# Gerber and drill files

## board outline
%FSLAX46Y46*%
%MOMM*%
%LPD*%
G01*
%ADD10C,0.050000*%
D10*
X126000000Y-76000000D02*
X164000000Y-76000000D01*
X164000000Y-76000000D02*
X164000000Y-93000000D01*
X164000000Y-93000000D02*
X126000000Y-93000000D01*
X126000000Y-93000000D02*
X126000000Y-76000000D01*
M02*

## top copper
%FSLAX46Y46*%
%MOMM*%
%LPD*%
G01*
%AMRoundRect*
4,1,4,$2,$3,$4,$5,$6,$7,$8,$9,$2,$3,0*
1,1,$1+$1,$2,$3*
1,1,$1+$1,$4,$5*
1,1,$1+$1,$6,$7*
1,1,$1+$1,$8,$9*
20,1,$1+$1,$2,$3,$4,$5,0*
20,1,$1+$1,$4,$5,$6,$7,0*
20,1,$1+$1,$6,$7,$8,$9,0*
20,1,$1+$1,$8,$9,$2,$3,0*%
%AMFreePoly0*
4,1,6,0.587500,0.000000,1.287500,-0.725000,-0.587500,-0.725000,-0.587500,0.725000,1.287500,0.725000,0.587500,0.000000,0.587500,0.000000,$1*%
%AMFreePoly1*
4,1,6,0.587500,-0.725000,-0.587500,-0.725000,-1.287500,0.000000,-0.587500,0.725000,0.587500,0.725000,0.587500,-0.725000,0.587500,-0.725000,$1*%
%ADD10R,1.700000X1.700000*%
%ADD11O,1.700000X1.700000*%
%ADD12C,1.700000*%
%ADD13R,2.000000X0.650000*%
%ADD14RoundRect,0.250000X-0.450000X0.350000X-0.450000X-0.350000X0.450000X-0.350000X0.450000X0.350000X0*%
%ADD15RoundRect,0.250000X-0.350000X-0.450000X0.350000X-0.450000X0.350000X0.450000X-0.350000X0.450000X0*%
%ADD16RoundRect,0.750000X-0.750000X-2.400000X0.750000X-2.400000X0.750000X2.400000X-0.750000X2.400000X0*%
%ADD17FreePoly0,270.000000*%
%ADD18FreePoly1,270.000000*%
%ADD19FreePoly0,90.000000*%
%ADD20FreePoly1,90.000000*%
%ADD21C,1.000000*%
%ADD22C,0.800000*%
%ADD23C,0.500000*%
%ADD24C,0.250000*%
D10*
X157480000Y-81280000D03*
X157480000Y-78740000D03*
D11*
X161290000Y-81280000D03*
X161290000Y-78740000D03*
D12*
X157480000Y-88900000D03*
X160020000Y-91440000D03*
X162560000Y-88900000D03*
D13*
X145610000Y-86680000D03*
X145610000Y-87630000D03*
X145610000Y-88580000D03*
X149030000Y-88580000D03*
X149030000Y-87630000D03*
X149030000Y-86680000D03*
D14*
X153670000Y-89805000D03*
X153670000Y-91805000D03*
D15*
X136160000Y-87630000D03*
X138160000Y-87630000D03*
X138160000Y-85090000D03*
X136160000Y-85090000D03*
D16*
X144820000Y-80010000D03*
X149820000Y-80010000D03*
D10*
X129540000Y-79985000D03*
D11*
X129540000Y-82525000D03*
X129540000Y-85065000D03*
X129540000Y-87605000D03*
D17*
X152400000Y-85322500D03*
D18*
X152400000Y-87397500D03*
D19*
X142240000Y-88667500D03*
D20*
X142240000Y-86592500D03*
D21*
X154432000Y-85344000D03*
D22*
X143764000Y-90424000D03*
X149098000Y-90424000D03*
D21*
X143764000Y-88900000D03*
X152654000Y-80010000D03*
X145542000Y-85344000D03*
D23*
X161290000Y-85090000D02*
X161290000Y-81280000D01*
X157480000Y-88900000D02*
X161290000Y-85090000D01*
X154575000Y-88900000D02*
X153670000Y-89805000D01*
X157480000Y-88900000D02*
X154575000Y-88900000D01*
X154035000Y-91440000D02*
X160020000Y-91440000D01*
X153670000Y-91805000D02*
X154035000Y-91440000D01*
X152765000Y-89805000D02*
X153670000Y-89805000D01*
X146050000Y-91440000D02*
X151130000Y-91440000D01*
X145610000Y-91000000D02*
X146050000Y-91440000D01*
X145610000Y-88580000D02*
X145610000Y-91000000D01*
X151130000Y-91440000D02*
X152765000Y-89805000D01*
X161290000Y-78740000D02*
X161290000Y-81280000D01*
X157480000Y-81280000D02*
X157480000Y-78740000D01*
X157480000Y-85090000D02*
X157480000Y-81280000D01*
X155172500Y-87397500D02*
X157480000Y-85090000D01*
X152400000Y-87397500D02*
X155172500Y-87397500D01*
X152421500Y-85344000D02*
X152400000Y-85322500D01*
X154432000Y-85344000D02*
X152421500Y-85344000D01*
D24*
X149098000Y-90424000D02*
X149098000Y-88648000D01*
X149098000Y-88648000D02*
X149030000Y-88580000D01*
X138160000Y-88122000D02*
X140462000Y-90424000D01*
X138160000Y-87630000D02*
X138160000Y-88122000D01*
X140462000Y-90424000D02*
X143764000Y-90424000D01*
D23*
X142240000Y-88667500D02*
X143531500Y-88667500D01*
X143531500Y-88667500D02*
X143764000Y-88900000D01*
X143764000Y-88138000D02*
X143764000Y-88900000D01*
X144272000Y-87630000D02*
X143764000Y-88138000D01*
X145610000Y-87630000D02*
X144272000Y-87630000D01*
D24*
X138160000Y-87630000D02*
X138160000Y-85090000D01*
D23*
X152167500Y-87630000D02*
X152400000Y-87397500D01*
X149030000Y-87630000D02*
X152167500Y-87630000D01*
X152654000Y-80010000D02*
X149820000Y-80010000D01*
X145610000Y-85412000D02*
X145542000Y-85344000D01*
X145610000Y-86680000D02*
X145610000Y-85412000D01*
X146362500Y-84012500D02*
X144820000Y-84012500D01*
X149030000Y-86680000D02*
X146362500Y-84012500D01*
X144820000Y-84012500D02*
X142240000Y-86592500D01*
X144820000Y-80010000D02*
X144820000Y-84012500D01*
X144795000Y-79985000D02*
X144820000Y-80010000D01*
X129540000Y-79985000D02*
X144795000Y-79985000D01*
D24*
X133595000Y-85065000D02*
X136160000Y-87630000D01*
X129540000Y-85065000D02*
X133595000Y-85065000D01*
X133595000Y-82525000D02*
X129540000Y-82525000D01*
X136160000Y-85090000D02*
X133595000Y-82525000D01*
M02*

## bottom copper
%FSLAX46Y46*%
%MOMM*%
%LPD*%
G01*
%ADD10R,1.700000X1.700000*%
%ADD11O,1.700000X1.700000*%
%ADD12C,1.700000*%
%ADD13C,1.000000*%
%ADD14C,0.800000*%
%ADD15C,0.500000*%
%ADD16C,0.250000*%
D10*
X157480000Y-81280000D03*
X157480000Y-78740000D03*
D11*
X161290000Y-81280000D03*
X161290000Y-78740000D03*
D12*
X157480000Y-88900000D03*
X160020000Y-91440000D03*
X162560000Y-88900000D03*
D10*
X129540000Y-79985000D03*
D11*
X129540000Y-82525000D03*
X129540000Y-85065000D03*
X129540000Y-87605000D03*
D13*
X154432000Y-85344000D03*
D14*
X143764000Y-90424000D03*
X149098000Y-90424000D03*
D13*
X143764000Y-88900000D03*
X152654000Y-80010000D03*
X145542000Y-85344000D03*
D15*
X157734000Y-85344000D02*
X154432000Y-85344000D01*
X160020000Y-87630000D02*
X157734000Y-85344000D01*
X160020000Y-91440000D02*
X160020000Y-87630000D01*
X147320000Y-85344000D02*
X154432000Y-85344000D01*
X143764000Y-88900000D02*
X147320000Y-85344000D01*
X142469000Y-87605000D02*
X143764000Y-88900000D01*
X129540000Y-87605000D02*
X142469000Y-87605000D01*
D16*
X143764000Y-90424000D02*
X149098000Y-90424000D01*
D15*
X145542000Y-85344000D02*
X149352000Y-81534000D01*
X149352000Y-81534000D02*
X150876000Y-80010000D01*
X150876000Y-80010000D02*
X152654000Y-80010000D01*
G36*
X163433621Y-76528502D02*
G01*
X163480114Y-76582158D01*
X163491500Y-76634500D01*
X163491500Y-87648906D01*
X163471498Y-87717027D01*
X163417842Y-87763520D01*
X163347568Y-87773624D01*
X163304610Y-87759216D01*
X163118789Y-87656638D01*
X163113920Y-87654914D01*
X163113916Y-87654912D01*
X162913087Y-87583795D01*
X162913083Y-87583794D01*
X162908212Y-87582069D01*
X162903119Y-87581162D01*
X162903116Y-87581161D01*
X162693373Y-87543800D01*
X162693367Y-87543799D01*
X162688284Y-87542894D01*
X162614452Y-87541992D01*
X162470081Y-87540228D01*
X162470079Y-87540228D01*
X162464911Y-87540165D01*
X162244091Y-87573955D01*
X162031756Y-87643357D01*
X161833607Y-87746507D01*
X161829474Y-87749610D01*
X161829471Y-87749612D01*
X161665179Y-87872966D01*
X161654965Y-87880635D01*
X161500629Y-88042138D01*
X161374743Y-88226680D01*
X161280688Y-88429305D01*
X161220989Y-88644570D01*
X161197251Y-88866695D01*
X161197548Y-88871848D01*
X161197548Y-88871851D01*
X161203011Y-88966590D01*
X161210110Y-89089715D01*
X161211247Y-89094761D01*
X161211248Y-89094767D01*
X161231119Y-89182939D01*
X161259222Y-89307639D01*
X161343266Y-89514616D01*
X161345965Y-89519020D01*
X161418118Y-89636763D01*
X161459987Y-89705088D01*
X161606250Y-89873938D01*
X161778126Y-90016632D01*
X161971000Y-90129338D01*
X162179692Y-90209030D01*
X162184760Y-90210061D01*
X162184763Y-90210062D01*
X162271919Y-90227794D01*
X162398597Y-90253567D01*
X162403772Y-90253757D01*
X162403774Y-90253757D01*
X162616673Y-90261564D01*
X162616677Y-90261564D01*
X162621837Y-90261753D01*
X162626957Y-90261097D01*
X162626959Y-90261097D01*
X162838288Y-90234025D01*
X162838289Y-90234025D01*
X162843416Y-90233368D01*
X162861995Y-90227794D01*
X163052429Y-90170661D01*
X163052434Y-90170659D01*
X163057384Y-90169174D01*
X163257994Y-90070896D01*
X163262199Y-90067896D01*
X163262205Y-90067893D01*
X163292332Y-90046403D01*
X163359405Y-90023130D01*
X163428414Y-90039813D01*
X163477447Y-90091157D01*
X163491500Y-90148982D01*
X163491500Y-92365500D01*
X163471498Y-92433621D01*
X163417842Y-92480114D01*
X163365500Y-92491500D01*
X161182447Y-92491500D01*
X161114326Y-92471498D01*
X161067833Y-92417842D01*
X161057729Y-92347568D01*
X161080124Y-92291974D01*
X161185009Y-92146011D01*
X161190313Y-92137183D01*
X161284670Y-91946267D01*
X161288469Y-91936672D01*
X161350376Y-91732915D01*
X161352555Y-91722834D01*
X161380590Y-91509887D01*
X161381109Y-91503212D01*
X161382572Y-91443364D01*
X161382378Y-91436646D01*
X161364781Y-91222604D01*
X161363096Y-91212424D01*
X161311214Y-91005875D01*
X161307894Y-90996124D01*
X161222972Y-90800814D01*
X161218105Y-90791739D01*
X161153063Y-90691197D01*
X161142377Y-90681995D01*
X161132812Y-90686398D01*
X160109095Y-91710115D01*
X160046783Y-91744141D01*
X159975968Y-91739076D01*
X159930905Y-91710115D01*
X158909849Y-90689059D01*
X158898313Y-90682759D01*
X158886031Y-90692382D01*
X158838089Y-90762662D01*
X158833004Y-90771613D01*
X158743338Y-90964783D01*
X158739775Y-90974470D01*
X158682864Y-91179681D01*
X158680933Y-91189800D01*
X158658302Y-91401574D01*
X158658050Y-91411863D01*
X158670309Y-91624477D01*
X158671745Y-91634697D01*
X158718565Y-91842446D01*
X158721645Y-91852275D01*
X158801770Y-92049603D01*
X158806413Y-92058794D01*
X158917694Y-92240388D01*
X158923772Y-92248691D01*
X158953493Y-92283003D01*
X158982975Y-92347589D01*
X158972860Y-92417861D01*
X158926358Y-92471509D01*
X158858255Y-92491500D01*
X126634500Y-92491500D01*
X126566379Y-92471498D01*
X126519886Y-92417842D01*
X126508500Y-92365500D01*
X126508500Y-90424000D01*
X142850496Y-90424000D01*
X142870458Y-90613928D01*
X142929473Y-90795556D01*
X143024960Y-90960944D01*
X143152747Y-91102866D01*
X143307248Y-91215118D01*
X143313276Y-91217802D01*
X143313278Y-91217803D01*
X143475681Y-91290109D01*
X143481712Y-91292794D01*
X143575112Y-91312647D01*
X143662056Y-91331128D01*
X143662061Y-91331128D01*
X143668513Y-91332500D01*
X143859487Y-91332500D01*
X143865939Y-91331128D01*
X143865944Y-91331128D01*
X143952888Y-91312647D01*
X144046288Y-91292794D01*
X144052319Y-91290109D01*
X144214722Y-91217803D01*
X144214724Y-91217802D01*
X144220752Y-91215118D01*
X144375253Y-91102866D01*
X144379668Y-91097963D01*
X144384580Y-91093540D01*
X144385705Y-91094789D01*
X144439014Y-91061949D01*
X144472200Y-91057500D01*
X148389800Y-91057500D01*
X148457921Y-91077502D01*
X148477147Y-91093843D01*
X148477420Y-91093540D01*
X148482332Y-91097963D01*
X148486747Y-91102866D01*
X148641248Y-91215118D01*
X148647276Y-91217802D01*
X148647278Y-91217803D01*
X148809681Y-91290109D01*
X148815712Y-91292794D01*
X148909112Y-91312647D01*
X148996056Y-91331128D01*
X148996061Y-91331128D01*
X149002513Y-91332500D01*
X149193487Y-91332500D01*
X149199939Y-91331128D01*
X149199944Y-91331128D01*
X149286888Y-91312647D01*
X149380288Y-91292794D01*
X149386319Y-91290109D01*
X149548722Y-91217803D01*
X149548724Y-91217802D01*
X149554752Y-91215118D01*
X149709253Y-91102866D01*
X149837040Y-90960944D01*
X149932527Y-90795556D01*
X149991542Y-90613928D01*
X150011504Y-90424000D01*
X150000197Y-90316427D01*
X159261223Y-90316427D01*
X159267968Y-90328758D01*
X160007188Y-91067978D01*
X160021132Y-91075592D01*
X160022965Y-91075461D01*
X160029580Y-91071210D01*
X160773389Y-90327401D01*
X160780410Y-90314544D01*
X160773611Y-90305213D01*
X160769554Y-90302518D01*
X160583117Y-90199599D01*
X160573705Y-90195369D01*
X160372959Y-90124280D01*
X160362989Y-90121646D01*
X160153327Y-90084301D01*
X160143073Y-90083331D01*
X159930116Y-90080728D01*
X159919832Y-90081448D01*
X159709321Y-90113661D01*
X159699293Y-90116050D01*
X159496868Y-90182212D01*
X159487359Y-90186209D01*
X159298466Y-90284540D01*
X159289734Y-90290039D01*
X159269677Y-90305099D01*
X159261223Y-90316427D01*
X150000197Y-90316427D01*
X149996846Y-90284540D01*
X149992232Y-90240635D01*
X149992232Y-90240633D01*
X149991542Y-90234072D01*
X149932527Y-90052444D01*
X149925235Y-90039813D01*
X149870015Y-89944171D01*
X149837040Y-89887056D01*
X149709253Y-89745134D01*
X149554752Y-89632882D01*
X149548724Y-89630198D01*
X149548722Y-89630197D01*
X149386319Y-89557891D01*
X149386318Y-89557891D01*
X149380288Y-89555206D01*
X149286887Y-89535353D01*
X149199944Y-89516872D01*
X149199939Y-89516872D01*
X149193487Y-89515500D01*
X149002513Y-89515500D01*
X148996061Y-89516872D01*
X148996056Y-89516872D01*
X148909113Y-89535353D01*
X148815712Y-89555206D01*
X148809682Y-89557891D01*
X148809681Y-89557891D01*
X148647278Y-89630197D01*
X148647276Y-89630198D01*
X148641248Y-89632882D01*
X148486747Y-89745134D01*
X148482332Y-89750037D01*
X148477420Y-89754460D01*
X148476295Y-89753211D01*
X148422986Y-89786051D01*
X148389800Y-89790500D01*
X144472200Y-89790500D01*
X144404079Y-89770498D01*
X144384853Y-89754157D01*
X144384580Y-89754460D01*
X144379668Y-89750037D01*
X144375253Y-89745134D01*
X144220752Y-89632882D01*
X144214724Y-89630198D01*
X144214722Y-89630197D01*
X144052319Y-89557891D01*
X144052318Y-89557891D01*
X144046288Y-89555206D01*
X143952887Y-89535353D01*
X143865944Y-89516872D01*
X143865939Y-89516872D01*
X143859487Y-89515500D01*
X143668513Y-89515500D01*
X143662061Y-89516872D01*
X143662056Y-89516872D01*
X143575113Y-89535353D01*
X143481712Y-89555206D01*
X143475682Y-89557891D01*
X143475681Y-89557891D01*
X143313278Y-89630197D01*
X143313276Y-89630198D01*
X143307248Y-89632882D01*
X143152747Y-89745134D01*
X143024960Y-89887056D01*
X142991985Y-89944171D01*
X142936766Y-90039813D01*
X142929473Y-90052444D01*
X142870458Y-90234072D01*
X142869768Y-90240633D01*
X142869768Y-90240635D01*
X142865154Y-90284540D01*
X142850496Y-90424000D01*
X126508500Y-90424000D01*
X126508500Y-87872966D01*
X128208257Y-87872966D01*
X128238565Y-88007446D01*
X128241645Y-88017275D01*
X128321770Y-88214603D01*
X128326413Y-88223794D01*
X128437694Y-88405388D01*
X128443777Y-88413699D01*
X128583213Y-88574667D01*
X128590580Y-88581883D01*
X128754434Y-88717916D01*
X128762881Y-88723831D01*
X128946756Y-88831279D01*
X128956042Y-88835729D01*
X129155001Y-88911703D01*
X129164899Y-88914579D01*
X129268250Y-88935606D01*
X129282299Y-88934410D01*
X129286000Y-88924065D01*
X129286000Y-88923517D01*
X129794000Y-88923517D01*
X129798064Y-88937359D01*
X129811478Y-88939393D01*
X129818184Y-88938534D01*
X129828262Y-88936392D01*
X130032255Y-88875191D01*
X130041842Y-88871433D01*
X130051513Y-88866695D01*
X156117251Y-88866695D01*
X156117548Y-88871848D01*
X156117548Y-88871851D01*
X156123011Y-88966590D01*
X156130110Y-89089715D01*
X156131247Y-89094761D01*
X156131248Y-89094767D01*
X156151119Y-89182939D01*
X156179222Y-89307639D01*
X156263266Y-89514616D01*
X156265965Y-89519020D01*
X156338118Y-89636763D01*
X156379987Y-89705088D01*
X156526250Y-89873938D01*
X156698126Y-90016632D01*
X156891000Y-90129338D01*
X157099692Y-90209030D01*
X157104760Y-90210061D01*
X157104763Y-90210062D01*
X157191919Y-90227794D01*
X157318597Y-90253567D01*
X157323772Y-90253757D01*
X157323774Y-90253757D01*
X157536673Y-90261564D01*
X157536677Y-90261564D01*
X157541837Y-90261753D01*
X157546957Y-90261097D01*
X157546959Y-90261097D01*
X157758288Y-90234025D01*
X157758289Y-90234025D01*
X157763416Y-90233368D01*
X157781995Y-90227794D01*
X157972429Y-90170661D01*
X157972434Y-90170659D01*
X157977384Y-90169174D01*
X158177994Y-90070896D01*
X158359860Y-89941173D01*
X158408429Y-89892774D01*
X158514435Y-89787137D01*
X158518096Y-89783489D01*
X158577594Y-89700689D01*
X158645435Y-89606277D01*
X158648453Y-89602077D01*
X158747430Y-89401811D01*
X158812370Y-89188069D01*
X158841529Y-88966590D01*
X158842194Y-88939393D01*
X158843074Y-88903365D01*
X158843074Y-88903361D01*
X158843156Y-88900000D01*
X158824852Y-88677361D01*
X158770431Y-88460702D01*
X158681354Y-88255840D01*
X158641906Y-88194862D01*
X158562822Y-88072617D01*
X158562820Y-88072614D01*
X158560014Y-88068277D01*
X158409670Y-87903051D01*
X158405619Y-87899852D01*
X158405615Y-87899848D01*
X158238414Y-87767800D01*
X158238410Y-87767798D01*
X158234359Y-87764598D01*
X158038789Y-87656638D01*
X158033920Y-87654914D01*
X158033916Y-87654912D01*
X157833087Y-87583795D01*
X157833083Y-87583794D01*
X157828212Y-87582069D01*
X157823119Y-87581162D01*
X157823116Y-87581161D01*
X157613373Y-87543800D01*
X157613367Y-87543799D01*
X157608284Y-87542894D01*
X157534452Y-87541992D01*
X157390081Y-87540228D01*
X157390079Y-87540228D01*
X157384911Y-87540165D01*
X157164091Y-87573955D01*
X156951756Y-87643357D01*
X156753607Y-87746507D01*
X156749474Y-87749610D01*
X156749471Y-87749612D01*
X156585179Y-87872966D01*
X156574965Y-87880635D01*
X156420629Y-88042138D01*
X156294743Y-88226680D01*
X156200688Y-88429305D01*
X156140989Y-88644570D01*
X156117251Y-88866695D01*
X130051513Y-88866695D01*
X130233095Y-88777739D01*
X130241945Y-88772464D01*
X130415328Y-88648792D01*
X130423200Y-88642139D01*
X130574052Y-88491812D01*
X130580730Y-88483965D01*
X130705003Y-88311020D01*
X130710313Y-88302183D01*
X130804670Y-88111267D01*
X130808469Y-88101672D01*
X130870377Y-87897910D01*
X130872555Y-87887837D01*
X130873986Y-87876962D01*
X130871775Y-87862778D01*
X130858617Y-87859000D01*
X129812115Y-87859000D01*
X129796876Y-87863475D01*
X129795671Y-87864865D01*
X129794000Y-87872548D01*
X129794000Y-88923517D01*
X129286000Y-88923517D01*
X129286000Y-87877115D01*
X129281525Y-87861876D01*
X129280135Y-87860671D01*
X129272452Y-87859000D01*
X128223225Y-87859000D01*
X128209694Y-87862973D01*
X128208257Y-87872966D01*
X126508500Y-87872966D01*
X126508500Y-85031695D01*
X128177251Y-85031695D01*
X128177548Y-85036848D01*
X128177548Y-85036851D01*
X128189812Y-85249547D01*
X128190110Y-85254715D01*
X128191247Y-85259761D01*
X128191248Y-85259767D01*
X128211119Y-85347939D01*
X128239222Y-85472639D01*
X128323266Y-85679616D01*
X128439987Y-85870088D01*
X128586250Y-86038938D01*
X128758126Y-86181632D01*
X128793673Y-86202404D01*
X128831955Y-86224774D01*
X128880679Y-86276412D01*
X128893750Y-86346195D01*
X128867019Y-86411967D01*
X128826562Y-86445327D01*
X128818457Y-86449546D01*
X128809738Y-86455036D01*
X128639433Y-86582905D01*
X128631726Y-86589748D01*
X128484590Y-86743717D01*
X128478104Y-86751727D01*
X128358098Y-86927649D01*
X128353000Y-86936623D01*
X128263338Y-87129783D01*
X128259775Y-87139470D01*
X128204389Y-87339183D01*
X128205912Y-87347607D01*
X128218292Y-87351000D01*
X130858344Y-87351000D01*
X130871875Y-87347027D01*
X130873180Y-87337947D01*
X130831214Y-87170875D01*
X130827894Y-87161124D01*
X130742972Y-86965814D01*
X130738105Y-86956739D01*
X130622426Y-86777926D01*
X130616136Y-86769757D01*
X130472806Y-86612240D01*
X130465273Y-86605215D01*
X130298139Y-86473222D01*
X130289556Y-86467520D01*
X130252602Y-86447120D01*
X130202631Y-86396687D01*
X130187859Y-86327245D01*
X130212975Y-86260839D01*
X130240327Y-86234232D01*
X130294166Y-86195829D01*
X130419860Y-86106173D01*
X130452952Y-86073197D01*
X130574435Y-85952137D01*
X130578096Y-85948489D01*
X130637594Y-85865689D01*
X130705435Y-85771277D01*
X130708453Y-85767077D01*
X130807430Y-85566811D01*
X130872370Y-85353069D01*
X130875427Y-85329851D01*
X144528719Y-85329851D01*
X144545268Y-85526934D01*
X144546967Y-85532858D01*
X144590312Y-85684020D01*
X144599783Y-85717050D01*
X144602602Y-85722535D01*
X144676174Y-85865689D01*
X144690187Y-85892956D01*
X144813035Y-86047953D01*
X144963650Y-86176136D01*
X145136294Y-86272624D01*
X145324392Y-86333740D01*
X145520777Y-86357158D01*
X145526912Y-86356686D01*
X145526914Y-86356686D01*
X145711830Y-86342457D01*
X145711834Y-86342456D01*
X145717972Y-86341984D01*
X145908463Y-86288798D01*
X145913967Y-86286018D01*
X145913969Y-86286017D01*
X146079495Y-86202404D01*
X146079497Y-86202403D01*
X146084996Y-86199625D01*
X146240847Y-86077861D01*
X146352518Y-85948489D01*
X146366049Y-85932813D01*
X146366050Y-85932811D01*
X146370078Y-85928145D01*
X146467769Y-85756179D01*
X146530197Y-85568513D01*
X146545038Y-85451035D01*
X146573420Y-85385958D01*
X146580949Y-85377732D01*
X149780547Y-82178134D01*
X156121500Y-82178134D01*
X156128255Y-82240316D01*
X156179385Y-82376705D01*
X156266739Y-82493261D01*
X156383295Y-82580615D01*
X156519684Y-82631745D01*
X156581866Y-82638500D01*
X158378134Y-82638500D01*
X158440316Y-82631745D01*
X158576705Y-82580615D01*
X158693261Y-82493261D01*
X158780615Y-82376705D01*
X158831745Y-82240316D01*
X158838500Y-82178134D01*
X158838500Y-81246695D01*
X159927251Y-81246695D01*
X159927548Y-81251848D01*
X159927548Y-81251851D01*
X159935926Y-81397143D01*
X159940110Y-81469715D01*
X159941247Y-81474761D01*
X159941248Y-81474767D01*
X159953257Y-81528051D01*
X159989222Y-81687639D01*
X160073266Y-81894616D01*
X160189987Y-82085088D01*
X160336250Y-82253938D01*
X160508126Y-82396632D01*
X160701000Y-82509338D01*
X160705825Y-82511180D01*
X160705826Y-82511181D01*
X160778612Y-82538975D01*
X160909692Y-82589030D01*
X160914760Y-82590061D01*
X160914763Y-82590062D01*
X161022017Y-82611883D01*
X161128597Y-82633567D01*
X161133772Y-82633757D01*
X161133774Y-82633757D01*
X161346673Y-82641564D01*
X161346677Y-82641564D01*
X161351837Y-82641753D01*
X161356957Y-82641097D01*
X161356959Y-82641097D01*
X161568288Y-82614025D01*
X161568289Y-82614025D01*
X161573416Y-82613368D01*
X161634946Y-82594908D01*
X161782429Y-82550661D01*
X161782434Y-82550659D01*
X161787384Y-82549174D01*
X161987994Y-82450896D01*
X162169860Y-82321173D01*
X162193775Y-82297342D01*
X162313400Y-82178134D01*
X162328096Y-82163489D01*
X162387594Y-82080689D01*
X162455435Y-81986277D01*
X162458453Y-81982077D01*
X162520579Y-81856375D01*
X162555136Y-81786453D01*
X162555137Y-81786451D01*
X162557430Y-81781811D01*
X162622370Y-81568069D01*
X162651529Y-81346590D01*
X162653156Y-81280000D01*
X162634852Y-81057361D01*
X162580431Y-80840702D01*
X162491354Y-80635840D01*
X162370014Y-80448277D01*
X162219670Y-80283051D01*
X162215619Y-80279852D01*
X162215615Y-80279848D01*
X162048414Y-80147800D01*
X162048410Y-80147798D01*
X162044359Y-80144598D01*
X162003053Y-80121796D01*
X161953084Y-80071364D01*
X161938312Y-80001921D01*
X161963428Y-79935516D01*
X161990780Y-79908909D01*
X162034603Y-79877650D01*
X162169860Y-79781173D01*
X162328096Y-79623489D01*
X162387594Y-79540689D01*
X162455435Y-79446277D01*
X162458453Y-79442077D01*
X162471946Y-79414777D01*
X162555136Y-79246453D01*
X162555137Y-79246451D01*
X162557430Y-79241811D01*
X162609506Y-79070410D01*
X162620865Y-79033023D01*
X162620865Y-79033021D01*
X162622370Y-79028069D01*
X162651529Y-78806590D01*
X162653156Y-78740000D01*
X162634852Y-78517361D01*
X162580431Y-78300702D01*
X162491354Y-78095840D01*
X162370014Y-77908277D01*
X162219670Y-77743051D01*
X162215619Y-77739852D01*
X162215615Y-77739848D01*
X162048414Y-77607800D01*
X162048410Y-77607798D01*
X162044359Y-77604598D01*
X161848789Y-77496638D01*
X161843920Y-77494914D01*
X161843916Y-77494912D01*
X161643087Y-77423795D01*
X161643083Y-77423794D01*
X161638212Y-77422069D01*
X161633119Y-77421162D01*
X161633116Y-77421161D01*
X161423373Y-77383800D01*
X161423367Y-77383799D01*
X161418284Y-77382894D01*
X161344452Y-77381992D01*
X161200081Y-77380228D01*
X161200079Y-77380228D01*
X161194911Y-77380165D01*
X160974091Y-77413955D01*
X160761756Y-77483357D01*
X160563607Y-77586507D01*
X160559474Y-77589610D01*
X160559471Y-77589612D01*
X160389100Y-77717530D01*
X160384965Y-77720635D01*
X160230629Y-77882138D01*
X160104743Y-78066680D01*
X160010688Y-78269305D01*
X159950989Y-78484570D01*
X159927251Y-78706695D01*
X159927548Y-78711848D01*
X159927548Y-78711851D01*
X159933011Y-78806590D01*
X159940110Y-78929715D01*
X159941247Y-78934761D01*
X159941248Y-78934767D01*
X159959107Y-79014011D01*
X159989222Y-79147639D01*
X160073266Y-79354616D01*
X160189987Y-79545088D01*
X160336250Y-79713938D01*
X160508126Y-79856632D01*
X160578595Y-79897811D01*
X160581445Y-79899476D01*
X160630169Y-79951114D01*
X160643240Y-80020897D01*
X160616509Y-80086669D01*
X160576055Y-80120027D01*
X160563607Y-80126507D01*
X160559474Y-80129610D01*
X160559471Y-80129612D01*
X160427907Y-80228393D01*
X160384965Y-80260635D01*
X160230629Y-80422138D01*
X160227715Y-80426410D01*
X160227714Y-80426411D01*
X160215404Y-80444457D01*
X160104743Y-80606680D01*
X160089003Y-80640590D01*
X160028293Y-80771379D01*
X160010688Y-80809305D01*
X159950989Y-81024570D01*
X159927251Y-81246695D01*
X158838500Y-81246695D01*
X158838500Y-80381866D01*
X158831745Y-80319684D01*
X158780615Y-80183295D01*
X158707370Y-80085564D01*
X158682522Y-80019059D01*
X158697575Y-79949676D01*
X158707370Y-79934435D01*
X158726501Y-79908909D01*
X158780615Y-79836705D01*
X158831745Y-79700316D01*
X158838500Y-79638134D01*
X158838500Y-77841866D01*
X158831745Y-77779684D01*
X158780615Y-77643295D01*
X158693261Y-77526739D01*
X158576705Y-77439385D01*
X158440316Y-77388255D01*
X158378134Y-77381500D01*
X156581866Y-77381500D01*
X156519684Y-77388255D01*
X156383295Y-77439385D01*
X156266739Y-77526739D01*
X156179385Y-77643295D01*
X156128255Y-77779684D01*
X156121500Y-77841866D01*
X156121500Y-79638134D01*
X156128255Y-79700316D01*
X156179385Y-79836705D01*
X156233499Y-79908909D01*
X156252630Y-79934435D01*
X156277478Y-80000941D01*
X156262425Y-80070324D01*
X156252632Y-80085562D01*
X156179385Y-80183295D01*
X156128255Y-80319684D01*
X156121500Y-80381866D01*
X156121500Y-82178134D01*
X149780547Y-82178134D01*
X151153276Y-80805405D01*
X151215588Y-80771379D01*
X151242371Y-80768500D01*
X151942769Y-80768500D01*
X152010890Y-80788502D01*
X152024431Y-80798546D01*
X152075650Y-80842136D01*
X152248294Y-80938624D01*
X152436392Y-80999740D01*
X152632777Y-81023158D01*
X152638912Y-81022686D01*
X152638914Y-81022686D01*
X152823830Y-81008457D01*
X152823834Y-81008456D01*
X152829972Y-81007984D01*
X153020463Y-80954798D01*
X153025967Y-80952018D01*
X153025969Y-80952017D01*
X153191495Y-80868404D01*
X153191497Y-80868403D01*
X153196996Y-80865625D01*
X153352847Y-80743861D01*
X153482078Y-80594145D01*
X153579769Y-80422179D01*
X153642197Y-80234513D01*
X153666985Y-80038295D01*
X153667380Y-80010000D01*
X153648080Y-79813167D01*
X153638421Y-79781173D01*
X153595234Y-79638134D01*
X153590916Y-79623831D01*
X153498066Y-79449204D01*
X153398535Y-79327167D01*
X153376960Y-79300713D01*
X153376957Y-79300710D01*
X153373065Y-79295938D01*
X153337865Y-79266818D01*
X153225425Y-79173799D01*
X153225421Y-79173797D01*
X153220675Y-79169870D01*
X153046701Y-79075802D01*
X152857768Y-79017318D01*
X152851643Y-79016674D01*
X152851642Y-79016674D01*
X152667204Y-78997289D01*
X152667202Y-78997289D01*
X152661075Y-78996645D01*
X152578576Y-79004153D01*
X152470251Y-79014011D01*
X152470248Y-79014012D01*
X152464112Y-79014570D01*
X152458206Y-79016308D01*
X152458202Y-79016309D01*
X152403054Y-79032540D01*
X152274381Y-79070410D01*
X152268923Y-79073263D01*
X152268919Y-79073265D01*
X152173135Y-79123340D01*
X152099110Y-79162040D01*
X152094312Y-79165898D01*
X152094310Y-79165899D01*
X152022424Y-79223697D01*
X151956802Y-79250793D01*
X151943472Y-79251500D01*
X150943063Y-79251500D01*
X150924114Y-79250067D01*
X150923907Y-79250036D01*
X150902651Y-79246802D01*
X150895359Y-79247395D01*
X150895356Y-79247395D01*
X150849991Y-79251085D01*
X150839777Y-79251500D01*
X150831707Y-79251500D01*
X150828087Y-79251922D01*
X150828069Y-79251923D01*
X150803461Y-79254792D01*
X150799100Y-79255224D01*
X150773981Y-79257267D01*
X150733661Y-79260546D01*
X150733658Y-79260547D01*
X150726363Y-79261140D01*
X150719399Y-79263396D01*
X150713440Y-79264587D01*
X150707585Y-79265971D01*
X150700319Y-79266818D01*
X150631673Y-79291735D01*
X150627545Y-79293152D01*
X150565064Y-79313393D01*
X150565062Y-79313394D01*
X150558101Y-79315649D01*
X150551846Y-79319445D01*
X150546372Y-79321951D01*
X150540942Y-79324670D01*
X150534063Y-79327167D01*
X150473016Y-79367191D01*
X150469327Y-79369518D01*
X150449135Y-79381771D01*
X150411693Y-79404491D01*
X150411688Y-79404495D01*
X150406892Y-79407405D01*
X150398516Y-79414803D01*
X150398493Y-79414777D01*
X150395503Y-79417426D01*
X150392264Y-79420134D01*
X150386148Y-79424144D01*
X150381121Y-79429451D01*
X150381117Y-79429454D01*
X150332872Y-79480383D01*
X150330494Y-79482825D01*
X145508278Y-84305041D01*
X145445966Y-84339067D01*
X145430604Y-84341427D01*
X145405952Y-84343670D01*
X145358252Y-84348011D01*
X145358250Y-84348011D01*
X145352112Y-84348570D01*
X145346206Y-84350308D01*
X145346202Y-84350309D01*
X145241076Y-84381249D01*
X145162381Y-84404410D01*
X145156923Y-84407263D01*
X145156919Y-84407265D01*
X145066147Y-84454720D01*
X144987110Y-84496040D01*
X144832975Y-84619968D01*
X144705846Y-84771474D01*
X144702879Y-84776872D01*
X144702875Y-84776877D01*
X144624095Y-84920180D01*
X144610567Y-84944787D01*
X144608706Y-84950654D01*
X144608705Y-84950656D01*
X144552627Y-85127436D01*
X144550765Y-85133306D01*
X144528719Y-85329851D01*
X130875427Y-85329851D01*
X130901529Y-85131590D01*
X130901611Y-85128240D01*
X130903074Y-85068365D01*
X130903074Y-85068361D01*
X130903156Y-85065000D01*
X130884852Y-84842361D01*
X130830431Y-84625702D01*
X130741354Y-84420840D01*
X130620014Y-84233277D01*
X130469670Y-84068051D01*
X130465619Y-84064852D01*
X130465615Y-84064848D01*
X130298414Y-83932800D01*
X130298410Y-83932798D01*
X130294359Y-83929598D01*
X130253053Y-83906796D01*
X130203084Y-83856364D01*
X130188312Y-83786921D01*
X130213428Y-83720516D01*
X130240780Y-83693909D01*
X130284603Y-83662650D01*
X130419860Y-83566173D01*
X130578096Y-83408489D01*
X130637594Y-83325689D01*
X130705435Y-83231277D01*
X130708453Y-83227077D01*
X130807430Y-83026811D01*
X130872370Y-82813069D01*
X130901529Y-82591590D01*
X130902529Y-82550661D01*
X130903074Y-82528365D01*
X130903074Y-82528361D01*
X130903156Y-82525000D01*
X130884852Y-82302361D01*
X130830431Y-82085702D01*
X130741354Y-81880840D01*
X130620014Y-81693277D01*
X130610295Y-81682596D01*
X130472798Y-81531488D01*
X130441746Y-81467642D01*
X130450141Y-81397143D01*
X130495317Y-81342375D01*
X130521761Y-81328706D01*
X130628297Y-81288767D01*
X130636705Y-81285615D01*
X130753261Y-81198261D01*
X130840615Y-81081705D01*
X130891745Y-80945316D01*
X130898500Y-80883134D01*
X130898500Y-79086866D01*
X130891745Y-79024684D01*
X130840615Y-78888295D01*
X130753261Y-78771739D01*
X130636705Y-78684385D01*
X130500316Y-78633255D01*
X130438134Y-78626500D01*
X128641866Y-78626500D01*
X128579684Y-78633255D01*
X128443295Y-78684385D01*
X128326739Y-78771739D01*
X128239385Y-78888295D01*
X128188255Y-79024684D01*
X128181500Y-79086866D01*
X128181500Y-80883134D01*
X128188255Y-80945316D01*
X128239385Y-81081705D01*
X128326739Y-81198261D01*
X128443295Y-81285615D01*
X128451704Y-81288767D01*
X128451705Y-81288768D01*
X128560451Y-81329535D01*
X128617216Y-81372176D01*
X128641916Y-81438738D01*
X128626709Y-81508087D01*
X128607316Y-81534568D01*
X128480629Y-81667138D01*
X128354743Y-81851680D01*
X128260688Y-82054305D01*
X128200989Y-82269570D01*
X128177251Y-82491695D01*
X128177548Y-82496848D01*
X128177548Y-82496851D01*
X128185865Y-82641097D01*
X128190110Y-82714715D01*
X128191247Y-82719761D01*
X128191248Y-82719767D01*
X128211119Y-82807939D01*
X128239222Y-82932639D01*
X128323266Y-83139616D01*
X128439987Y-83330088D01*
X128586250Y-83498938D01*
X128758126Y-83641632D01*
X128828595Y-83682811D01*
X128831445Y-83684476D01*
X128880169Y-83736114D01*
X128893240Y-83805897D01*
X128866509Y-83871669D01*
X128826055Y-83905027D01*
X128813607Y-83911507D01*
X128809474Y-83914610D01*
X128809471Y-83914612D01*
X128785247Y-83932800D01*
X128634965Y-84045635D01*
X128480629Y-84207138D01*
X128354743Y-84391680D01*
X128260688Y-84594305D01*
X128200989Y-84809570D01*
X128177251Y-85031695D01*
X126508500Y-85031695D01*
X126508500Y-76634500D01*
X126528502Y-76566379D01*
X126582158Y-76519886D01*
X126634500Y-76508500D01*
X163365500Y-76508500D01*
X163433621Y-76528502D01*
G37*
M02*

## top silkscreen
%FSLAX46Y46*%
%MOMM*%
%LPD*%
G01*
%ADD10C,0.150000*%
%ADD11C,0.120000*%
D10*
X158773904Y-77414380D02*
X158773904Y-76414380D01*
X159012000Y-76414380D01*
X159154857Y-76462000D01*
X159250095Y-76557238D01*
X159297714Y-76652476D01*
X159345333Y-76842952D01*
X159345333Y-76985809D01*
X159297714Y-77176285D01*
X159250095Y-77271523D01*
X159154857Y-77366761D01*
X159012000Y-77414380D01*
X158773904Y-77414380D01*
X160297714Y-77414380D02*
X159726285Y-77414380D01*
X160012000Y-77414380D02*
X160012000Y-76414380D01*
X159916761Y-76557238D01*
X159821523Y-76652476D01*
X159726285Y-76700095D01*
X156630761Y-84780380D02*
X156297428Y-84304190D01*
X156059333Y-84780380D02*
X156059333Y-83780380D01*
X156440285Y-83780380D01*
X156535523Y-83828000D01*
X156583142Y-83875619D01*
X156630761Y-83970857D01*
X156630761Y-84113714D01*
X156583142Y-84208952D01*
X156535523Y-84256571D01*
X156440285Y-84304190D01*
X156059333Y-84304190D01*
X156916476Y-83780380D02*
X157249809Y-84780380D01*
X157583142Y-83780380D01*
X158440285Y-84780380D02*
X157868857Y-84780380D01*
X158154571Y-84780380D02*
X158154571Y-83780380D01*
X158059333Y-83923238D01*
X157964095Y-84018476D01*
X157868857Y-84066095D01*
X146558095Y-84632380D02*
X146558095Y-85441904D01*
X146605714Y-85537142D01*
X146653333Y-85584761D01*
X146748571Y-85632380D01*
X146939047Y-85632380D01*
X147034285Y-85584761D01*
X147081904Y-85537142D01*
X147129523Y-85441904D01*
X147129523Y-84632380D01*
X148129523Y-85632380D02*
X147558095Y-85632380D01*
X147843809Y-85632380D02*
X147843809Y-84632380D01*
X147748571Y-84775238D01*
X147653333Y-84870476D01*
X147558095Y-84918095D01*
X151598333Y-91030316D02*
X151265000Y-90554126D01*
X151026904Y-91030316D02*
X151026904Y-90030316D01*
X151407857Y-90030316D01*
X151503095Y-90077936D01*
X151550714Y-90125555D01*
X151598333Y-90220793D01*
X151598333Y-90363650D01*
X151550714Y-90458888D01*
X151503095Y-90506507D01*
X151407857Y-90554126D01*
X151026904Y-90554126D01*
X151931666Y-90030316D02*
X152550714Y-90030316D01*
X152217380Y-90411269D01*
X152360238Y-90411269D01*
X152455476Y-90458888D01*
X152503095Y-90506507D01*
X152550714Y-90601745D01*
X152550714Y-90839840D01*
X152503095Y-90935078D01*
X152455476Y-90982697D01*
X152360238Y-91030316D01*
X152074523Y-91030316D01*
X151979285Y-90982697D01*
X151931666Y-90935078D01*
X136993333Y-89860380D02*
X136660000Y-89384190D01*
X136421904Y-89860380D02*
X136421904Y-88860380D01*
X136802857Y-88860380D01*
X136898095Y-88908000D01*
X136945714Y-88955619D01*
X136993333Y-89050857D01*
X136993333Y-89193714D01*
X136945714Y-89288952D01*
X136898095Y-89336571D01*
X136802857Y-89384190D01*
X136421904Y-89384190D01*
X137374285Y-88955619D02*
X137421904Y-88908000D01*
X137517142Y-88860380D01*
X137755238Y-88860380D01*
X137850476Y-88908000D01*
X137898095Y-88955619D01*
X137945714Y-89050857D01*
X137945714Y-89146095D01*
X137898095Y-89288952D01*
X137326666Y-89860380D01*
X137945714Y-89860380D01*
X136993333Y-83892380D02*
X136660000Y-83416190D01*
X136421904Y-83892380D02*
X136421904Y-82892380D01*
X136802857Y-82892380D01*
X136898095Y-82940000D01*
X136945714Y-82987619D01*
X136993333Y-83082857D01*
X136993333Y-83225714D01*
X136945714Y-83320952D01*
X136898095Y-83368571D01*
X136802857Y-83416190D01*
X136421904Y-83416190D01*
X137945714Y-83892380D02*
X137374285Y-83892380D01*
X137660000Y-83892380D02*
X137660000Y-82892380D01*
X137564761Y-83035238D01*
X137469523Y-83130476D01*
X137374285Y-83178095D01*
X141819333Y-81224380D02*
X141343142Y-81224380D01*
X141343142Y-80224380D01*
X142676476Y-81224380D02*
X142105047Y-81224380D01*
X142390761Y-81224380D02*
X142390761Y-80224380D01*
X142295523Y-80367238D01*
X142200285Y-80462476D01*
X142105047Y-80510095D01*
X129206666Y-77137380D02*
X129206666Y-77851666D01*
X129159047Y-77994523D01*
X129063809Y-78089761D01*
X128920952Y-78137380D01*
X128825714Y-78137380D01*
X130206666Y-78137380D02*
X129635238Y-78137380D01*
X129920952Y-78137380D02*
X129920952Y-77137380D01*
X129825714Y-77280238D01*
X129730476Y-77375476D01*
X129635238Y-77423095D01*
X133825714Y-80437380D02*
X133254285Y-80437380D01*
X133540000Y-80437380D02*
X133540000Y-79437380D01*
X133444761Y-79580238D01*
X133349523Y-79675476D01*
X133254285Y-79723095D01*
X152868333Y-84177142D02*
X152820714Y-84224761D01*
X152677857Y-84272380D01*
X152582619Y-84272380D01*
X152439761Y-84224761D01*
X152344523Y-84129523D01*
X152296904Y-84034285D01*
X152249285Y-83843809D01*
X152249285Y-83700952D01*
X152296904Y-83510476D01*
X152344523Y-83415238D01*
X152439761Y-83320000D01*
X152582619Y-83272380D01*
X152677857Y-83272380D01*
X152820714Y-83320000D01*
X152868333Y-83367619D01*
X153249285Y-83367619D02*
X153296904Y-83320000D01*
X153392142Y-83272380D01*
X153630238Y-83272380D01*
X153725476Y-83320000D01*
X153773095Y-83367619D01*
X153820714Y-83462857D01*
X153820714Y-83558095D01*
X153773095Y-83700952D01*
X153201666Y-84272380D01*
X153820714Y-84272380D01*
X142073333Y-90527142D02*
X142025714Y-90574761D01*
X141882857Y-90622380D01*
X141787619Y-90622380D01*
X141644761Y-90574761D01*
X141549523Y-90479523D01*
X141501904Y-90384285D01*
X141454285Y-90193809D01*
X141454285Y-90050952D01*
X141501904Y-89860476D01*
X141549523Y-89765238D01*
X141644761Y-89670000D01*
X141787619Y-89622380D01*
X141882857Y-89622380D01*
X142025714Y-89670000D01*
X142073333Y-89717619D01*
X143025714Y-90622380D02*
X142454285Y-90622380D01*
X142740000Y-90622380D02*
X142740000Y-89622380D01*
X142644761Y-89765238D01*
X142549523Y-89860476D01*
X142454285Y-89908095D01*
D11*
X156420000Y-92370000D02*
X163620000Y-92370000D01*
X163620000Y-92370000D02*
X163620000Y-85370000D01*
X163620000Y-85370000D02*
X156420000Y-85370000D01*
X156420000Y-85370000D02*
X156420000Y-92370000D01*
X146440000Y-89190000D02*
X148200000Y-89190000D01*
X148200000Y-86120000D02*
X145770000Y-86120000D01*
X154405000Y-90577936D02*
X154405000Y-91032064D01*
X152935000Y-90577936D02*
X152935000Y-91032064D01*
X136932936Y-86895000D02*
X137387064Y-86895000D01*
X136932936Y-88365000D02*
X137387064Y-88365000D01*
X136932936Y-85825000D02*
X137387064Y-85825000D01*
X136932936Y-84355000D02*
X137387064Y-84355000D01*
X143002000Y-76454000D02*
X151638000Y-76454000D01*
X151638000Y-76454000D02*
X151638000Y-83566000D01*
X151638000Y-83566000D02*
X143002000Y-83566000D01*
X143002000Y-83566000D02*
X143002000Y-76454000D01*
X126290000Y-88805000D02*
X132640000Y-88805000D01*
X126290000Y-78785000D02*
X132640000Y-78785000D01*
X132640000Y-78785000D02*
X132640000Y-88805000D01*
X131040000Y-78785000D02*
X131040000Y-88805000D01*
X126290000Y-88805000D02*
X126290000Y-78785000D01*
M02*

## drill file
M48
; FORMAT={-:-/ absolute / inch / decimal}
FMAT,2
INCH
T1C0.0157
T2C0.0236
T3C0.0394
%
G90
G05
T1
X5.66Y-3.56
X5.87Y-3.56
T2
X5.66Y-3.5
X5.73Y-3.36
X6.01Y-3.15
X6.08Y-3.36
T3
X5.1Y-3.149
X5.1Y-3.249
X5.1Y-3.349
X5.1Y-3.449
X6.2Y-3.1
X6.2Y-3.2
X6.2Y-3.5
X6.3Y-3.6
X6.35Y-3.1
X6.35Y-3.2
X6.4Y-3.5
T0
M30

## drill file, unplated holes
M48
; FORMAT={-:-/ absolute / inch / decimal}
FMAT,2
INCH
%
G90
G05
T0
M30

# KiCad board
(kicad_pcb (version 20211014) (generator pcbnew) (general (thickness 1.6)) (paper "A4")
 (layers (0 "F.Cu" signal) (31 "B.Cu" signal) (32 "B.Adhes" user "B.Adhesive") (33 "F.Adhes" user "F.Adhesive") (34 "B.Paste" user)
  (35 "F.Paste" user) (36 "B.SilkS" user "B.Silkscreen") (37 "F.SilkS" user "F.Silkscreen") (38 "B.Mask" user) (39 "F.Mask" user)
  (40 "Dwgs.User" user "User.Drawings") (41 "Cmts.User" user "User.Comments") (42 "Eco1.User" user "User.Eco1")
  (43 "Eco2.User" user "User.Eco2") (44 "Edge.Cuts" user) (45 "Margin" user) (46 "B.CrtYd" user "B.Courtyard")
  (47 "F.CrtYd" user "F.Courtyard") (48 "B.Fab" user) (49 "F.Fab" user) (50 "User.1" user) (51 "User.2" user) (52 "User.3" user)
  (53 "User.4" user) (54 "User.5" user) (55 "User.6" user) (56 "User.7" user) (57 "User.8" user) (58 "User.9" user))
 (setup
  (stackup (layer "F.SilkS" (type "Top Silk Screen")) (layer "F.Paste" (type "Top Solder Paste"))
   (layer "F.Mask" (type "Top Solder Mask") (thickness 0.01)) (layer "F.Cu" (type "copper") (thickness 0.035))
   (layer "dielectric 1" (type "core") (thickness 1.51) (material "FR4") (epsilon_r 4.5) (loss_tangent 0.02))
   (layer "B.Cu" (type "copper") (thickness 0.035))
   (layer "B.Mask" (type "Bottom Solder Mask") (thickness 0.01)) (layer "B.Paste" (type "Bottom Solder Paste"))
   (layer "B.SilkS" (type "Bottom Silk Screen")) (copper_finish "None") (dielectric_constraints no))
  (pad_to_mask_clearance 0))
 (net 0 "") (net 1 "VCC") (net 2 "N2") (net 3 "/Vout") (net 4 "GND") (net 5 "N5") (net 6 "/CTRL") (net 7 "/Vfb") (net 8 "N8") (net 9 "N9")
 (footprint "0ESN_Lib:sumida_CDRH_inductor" (layer "F.Cu") (at 147.32 80.01)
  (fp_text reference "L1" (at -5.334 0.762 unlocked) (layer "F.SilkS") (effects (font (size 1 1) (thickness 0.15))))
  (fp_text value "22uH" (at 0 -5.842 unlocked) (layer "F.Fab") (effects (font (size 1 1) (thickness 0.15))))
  (fp_rect (start -4.318 -3.556) (end 4.318 3.556) (layer "F.SilkS") (width 0.12) (fill none))
  (pad "1" smd roundrect (at -2.5 0) (size 3 6.3) (layers "F.Cu" "F.Paste" "F.Mask") (roundrect_rratio 0.25) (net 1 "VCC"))
  (pad "2" smd roundrect (at 2.5 0) (size 3 6.3) (layers "F.Cu" "F.Paste" "F.Mask") (roundrect_rratio 0.25) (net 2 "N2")))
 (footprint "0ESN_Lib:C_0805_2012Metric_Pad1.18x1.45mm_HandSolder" (layer "F.Cu") (at 152.4 86.36 90)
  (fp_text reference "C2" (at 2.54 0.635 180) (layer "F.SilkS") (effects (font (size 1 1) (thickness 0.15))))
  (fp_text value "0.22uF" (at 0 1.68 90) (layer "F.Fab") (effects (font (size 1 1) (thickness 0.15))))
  (pad "1" smd custom (at -1.0375 0 270) (size 1.175 1.45) (layers "F.Cu" "F.Paste" "F.Mask") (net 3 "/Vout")
   (options (clearance outline) (anchor rect)) (primitives))
  (pad "2" smd custom (at 1.0375 0 270) (size 1.175 1.45) (layers "F.Cu" "F.Paste" "F.Mask") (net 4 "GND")
   (options (clearance outline) (anchor rect)) (primitives)))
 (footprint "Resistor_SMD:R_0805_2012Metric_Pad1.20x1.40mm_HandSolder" (layer "F.Cu") (at 137.16 87.63)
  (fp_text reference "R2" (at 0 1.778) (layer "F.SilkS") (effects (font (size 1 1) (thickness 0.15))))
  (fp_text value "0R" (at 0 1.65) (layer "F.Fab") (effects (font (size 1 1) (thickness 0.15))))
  (fp_line (start -0.227064 0.735) (end 0.227064 0.735) (layer "F.SilkS") (width 0.12))
  (fp_line (start -0.227064 -0.735) (end 0.227064 -0.735) (layer "F.SilkS") (width 0.12))
  (pad "1" smd roundrect (at -1 0) (size 1.2 1.4) (layers "F.Cu" "F.Paste" "F.Mask") (roundrect_rratio 0.2083333333) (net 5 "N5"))
  (pad "2" smd roundrect (at 1 0) (size 1.2 1.4) (layers "F.Cu" "F.Paste" "F.Mask") (roundrect_rratio 0.2083333333) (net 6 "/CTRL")))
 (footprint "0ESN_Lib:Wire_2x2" (layer "F.Cu") (at 158.75 81.28 90)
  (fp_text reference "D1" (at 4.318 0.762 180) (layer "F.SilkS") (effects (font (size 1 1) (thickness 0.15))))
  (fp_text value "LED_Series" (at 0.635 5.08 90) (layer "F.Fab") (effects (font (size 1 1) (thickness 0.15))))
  (pad "1" thru_hole rect (at 0 -1.27 90) (size 1.7 1.7) (drill 1) (layers *.Cu *.Mask) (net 3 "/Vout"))
  (pad "1" thru_hole rect (at 2.54 -1.27 90) (size 1.7 1.7) (drill 1) (layers *.Cu *.Mask) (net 3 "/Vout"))
  (pad "2" thru_hole oval (at 2.54 2.54 90) (size 1.7 1.7) (drill 1) (layers *.Cu *.Mask) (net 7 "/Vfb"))
  (pad "2" thru_hole oval (at 0 2.54 90) (size 1.7 1.7) (drill 1) (layers *.Cu *.Mask) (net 7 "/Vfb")))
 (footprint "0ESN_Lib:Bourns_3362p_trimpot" (layer "F.Cu") (at 160.02 88.9)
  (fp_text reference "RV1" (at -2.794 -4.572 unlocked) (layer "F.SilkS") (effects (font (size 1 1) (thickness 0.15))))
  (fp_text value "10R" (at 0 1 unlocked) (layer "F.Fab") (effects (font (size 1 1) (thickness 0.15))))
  (fp_rect (start -3.6 3.47) (end 3.6 -3.53) (layer "F.SilkS") (width 0.12) (fill none))
  (pad "1" thru_hole circle (at -2.54 0) (size 1.7 1.7) (drill 1) (layers *.Cu *.Mask) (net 7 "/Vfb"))
  (pad "2" thru_hole circle (at 0 2.54) (size 1.7 1.7) (drill 1) (layers *.Cu *.Mask) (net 4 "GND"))
  (pad "3" thru_hole circle (at 2.54 0) (size 1.7 1.7) (drill 1) (layers *.Cu *.Mask) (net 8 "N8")))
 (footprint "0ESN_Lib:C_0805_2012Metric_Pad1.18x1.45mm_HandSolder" (layer "F.Cu") (at 142.24 87.63 -90)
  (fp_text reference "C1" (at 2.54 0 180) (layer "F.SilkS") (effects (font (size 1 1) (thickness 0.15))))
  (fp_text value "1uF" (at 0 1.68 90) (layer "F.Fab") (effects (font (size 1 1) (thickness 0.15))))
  (pad "1" smd custom (at -1.0375 0 90) (size 1.175 1.45) (layers "F.Cu" "F.Paste" "F.Mask") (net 1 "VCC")
   (options (clearance outline) (anchor rect)) (primitives))
  (pad "2" smd custom (at 1.0375 0 90) (size 1.175 1.45) (layers "F.Cu" "F.Paste" "F.Mask") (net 4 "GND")
   (options (clearance outline) (anchor rect)) (primitives)))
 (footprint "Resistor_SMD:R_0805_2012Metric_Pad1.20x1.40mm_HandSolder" (layer "F.Cu") (at 153.67 90.805 -90)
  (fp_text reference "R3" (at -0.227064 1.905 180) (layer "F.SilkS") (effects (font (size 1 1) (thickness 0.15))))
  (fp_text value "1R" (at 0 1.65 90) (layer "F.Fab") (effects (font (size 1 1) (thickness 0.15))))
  (fp_line (start -0.227064 -0.735) (end 0.227064 -0.735) (layer "F.SilkS") (width 0.12))
  (fp_line (start -0.227064 0.735) (end 0.227064 0.735) (layer "F.SilkS") (width 0.12))
  (pad "1" smd roundrect (at -1 0 270) (size 1.2 1.4) (layers "F.Cu" "F.Paste" "F.Mask") (roundrect_rratio 0.2083333333) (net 7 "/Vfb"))
  (pad "2" smd roundrect (at 1 0 270) (size 1.2 1.4) (layers "F.Cu" "F.Paste" "F.Mask") (roundrect_rratio 0.2083333333) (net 4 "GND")))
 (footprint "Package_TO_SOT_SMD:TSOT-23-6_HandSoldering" (layer "F.Cu") (at 147.32 87.63)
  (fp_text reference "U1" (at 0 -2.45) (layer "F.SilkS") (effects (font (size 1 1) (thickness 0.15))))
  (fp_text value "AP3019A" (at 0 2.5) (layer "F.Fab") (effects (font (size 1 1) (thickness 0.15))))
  (fp_line (start 0.88 -1.51) (end -1.55 -1.51) (layer "F.SilkS") (width 0.12))
  (fp_line (start -0.88 1.56) (end 0.88 1.56) (layer "F.SilkS") (width 0.12))
  (pad "1" smd rect (at -1.71 -0.95) (size 2 0.65) (layers "F.Cu" "F.Paste" "F.Mask") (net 2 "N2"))
  (pad "2" smd rect (at -1.71 0) (size 2 0.65) (layers "F.Cu" "F.Paste" "F.Mask") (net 4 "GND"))
  (pad "3" smd rect (at -1.71 0.95) (size 2 0.65) (layers "F.Cu" "F.Paste" "F.Mask") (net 7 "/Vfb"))
  (pad "4" smd rect (at 1.71 0.95) (size 2 0.65) (layers "F.Cu" "F.Paste" "F.Mask") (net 6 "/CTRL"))
  (pad "5" smd rect (at 1.71 0) (size 2 0.65) (layers "F.Cu" "F.Paste" "F.Mask") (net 3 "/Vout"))
  (pad "6" smd rect (at 1.71 -0.95) (size 2 0.65) (layers "F.Cu" "F.Paste" "F.Mask") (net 1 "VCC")))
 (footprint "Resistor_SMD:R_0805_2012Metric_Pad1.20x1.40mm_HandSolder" (layer "F.Cu") (at 137.16 85.09)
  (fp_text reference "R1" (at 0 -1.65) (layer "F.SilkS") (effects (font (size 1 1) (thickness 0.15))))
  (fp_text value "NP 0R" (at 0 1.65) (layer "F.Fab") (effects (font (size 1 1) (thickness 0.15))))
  (fp_line (start -0.227064 0.735) (end 0.227064 0.735) (layer "F.SilkS") (width 0.12))
  (fp_line (start -0.227064 -0.735) (end 0.227064 -0.735) (layer "F.SilkS") (width 0.12))
  (pad "1" smd roundrect (at -1 0) (size 1.2 1.4) (layers "F.Cu" "F.Paste" "F.Mask") (roundrect_rratio 0.2083333333) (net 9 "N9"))
  (pad "2" smd roundrect (at 1 0) (size 1.2 1.4) (layers "F.Cu" "F.Paste" "F.Mask") (roundrect_rratio 0.2083333333) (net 6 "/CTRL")))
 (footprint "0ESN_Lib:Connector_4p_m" (layer "F.Cu") (at 129.54 79.985)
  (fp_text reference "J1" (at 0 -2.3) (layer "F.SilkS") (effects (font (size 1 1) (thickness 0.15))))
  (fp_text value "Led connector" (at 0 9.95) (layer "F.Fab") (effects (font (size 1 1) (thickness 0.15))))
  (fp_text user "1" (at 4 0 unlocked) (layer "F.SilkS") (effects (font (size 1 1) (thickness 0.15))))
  (fp_line (start 1.5 -1.2) (end 1.5 8.82) (layer "F.SilkS") (width 0.12))
  (fp_line (start -3.25 8.82) (end -3.25 -1.2) (layer "F.SilkS") (width 0.12))
  (fp_line (start 3.1 -1.2) (end 3.1 8.82) (layer "F.SilkS") (width 0.12))
  (fp_line (start -3.25 -1.2) (end 3.1 -1.2) (layer "F.SilkS") (width 0.12))
  (fp_line (start -3.25 8.82) (end 3.1 8.82) (layer "F.SilkS") (width 0.12))
  (pad "1" thru_hole rect (at 0 0) (size 1.7 1.7) (drill 1) (layers *.Cu *.Mask) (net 1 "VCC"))
  (pad "2" thru_hole oval (at 0 2.54) (size 1.7 1.7) (drill 1) (layers *.Cu *.Mask) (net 9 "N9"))
  (pad "3" thru_hole oval (at 0 5.08) (size 1.7 1.7) (drill 1) (layers *.Cu *.Mask) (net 5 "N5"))
  (pad "4" thru_hole oval (at 0 7.62) (size 1.7 1.7) (drill 1) (layers *.Cu *.Mask) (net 4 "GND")))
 (gr_rect (start 126 76) (end 164 93) (layer "Edge.Cuts") (width 0.05) (fill none))
 (segment (start 129.54 79.985) (end 144.795 79.985) (width 0.5) (layer "F.Cu") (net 1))
 (segment (start 144.795 79.985) (end 144.82 80.01) (width 0.5) (layer "F.Cu") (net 1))
 (segment (start 149.03 86.68) (end 146.3625 84.0125) (width 0.5) (layer "F.Cu") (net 1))
 (segment (start 144.82 80.01) (end 144.82 84.0125) (width 0.5) (layer "F.Cu") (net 1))
 (segment (start 144.82 84.0125) (end 142.24 86.5925) (width 0.5) (layer "F.Cu") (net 1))
 (segment (start 146.3625 84.0125) (end 144.82 84.0125) (width 0.5) (layer "F.Cu") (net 1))
 (segment (start 154.035 91.44) (end 160.02 91.44) (width 0.5) (layer "F.Cu") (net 4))
 (segment (start 152.4215 85.344) (end 152.4 85.3225) (width 0.5) (layer "F.Cu") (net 4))
 (segment (start 145.61 87.63) (end 144.272 87.63) (width 0.5) (layer "F.Cu") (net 4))
 (segment (start 154.432 85.344) (end 152.4215 85.344) (width 0.5) (layer "F.Cu") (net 4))
 (segment (start 142.24 88.6675) (end 143.5315 88.6675) (width 0.5) (layer "F.Cu") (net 4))
 (segment (start 143.5315 88.6675) (end 143.764 88.9) (width 0.5) (layer "F.Cu") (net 4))
 (segment (start 153.67 91.805) (end 154.035 91.44) (width 0.5) (layer "F.Cu") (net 4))
 (segment (start 144.272 87.63) (end 143.764 88.138) (width 0.5) (layer "F.Cu") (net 4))
 (segment (start 143.764 88.138) (end 143.764 88.9) (width 0.5) (layer "F.Cu") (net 4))
 (via (at 143.764 88.9) (size 1) (drill 0.6) (layers "F.Cu" "B.Cu") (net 4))
 (via (at 154.432 85.344) (size 1) (drill 0.6) (layers "F.Cu" "B.Cu") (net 4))
 (segment (start 147.32 85.344) (end 154.432 85.344) (width 0.5) (layer "B.Cu") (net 4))
 (segment (start 157.734 85.344) (end 154.432 85.344) (width 0.5) (layer "B.Cu") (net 4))
 (segment (start 160.02 87.63) (end 157.734 85.344) (width 0.5) (layer "B.Cu") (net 4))
 (segment (start 142.469 87.605) (end 143.764 88.9) (width 0.5) (layer "B.Cu") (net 4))
 (segment (start 143.764 88.9) (end 147.32 85.344) (width 0.5) (layer "B.Cu") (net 4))
 (segment (start 129.54 87.605) (end 142.469 87.605) (width 0.5) (layer "B.Cu") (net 4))
 (segment (start 160.02 91.44) (end 160.02 87.63) (width 0.5) (layer "B.Cu") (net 4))
 (segment (start 152.4 87.3975) (end 155.1725 87.3975) (width 0.5) (layer "F.Cu") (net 3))
 (segment (start 157.48 81.28) (end 157.48 78.74) (width 0.5) (layer "F.Cu") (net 3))
 (segment (start 157.48 85.09) (end 157.48 81.28) (width 0.5) (layer "F.Cu") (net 3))
 (segment (start 155.1725 87.3975) (end 157.48 85.09) (width 0.5) (layer "F.Cu") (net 3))
 (segment (start 149.03 87.63) (end 152.1675 87.63) (width 0.5) (layer "F.Cu") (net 3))
 (segment (start 152.1675 87.63) (end 152.4 87.3975) (width 0.5) (layer "F.Cu") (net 3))
 (segment (start 157.48 88.9) (end 161.29 85.09) (width 0.5) (layer "F.Cu") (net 7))
 (segment (start 146.05 91.44) (end 151.13 91.44) (width 0.5) (layer "F.Cu") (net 7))
 (segment (start 145.61 91) (end 146.05 91.44) (width 0.5) (layer "F.Cu") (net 7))
 (segment (start 151.13 91.44) (end 152.765 89.805) (width 0.5) (layer "F.Cu") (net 7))
 (segment (start 154.575 88.9) (end 153.67 89.805) (width 0.5) (layer "F.Cu") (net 7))
 (segment (start 145.61 88.58) (end 145.61 91) (width 0.5) (layer "F.Cu") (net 7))
 (segment (start 152.765 89.805) (end 153.67 89.805) (width 0.5) (layer "F.Cu") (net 7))
 (segment (start 161.29 85.09) (end 161.29 81.28) (width 0.5) (layer "F.Cu") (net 7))
 (segment (start 161.29 78.74) (end 161.29 81.28) (width 0.5) (layer "F.Cu") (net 7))
 (segment (start 157.48 88.9) (end 154.575 88.9) (width 0.5) (layer "F.Cu") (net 7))
 (segment (start 136.16 85.09) (end 133.595 82.525) (width 0.25) (layer "F.Cu") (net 9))
 (segment (start 133.595 82.525) (end 129.54 82.525) (width 0.25) (layer "F.Cu") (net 9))
 (segment (start 133.595 85.065) (end 136.16 87.63) (width 0.25) (layer "F.Cu") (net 5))
 (segment (start 129.54 85.065) (end 133.595 85.065) (width 0.25) (layer "F.Cu") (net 5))
 (segment (start 145.61 86.68) (end 145.61 85.412) (width 0.5) (layer "F.Cu") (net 2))
 (segment (start 145.61 85.412) (end 145.542 85.344) (width 0.5) (layer "F.Cu") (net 2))
 (segment (start 152.654 80.01) (end 149.82 80.01) (width 0.5) (layer "F.Cu") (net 2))
 (via (at 145.542 85.344) (size 1) (drill 0.6) (layers "F.Cu" "B.Cu") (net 2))
 (via (at 152.654 80.01) (size 1) (drill 0.6) (layers "F.Cu" "B.Cu") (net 2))
 (segment (start 150.876 80.01) (end 152.654 80.01) (width 0.5) (layer "B.Cu") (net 2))
 (segment (start 145.542 85.344) (end 149.352 81.534) (width 0.5) (layer "B.Cu") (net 2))
 (segment (start 149.352 81.534) (end 150.876 80.01) (width 0.5) (layer "B.Cu") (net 2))
 (segment (start 138.16 87.63) (end 138.16 88.122) (width 0.25) (layer "F.Cu") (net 6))
 (segment (start 149.098 88.648) (end 149.03 88.58) (width 0.25) (layer "F.Cu") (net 6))
 (segment (start 140.462 90.424) (end 143.764 90.424) (width 0.25) (layer "F.Cu") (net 6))
 (segment (start 138.16 87.63) (end 138.16 85.09) (width 0.25) (layer "F.Cu") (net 6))
 (segment (start 138.16 88.122) (end 140.462 90.424) (width 0.25) (layer "F.Cu") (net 6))
 (segment (start 149.098 90.424) (end 149.098 88.648) (width 0.25) (layer "F.Cu") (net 6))
 (via (at 149.098 90.424) (size 0.8) (drill 0.4) (layers "F.Cu" "B.Cu") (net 6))
 (via (at 143.764 90.424) (size 0.8) (drill 0.4) (layers "F.Cu" "B.Cu") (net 6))
 (segment (start 143.764 90.424) (end 149.098 90.424) (width 0.25) (layer "B.Cu") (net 6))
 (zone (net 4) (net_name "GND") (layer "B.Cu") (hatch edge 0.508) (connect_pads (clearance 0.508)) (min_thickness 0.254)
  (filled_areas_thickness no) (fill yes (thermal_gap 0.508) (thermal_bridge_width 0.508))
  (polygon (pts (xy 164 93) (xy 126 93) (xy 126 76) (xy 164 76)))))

